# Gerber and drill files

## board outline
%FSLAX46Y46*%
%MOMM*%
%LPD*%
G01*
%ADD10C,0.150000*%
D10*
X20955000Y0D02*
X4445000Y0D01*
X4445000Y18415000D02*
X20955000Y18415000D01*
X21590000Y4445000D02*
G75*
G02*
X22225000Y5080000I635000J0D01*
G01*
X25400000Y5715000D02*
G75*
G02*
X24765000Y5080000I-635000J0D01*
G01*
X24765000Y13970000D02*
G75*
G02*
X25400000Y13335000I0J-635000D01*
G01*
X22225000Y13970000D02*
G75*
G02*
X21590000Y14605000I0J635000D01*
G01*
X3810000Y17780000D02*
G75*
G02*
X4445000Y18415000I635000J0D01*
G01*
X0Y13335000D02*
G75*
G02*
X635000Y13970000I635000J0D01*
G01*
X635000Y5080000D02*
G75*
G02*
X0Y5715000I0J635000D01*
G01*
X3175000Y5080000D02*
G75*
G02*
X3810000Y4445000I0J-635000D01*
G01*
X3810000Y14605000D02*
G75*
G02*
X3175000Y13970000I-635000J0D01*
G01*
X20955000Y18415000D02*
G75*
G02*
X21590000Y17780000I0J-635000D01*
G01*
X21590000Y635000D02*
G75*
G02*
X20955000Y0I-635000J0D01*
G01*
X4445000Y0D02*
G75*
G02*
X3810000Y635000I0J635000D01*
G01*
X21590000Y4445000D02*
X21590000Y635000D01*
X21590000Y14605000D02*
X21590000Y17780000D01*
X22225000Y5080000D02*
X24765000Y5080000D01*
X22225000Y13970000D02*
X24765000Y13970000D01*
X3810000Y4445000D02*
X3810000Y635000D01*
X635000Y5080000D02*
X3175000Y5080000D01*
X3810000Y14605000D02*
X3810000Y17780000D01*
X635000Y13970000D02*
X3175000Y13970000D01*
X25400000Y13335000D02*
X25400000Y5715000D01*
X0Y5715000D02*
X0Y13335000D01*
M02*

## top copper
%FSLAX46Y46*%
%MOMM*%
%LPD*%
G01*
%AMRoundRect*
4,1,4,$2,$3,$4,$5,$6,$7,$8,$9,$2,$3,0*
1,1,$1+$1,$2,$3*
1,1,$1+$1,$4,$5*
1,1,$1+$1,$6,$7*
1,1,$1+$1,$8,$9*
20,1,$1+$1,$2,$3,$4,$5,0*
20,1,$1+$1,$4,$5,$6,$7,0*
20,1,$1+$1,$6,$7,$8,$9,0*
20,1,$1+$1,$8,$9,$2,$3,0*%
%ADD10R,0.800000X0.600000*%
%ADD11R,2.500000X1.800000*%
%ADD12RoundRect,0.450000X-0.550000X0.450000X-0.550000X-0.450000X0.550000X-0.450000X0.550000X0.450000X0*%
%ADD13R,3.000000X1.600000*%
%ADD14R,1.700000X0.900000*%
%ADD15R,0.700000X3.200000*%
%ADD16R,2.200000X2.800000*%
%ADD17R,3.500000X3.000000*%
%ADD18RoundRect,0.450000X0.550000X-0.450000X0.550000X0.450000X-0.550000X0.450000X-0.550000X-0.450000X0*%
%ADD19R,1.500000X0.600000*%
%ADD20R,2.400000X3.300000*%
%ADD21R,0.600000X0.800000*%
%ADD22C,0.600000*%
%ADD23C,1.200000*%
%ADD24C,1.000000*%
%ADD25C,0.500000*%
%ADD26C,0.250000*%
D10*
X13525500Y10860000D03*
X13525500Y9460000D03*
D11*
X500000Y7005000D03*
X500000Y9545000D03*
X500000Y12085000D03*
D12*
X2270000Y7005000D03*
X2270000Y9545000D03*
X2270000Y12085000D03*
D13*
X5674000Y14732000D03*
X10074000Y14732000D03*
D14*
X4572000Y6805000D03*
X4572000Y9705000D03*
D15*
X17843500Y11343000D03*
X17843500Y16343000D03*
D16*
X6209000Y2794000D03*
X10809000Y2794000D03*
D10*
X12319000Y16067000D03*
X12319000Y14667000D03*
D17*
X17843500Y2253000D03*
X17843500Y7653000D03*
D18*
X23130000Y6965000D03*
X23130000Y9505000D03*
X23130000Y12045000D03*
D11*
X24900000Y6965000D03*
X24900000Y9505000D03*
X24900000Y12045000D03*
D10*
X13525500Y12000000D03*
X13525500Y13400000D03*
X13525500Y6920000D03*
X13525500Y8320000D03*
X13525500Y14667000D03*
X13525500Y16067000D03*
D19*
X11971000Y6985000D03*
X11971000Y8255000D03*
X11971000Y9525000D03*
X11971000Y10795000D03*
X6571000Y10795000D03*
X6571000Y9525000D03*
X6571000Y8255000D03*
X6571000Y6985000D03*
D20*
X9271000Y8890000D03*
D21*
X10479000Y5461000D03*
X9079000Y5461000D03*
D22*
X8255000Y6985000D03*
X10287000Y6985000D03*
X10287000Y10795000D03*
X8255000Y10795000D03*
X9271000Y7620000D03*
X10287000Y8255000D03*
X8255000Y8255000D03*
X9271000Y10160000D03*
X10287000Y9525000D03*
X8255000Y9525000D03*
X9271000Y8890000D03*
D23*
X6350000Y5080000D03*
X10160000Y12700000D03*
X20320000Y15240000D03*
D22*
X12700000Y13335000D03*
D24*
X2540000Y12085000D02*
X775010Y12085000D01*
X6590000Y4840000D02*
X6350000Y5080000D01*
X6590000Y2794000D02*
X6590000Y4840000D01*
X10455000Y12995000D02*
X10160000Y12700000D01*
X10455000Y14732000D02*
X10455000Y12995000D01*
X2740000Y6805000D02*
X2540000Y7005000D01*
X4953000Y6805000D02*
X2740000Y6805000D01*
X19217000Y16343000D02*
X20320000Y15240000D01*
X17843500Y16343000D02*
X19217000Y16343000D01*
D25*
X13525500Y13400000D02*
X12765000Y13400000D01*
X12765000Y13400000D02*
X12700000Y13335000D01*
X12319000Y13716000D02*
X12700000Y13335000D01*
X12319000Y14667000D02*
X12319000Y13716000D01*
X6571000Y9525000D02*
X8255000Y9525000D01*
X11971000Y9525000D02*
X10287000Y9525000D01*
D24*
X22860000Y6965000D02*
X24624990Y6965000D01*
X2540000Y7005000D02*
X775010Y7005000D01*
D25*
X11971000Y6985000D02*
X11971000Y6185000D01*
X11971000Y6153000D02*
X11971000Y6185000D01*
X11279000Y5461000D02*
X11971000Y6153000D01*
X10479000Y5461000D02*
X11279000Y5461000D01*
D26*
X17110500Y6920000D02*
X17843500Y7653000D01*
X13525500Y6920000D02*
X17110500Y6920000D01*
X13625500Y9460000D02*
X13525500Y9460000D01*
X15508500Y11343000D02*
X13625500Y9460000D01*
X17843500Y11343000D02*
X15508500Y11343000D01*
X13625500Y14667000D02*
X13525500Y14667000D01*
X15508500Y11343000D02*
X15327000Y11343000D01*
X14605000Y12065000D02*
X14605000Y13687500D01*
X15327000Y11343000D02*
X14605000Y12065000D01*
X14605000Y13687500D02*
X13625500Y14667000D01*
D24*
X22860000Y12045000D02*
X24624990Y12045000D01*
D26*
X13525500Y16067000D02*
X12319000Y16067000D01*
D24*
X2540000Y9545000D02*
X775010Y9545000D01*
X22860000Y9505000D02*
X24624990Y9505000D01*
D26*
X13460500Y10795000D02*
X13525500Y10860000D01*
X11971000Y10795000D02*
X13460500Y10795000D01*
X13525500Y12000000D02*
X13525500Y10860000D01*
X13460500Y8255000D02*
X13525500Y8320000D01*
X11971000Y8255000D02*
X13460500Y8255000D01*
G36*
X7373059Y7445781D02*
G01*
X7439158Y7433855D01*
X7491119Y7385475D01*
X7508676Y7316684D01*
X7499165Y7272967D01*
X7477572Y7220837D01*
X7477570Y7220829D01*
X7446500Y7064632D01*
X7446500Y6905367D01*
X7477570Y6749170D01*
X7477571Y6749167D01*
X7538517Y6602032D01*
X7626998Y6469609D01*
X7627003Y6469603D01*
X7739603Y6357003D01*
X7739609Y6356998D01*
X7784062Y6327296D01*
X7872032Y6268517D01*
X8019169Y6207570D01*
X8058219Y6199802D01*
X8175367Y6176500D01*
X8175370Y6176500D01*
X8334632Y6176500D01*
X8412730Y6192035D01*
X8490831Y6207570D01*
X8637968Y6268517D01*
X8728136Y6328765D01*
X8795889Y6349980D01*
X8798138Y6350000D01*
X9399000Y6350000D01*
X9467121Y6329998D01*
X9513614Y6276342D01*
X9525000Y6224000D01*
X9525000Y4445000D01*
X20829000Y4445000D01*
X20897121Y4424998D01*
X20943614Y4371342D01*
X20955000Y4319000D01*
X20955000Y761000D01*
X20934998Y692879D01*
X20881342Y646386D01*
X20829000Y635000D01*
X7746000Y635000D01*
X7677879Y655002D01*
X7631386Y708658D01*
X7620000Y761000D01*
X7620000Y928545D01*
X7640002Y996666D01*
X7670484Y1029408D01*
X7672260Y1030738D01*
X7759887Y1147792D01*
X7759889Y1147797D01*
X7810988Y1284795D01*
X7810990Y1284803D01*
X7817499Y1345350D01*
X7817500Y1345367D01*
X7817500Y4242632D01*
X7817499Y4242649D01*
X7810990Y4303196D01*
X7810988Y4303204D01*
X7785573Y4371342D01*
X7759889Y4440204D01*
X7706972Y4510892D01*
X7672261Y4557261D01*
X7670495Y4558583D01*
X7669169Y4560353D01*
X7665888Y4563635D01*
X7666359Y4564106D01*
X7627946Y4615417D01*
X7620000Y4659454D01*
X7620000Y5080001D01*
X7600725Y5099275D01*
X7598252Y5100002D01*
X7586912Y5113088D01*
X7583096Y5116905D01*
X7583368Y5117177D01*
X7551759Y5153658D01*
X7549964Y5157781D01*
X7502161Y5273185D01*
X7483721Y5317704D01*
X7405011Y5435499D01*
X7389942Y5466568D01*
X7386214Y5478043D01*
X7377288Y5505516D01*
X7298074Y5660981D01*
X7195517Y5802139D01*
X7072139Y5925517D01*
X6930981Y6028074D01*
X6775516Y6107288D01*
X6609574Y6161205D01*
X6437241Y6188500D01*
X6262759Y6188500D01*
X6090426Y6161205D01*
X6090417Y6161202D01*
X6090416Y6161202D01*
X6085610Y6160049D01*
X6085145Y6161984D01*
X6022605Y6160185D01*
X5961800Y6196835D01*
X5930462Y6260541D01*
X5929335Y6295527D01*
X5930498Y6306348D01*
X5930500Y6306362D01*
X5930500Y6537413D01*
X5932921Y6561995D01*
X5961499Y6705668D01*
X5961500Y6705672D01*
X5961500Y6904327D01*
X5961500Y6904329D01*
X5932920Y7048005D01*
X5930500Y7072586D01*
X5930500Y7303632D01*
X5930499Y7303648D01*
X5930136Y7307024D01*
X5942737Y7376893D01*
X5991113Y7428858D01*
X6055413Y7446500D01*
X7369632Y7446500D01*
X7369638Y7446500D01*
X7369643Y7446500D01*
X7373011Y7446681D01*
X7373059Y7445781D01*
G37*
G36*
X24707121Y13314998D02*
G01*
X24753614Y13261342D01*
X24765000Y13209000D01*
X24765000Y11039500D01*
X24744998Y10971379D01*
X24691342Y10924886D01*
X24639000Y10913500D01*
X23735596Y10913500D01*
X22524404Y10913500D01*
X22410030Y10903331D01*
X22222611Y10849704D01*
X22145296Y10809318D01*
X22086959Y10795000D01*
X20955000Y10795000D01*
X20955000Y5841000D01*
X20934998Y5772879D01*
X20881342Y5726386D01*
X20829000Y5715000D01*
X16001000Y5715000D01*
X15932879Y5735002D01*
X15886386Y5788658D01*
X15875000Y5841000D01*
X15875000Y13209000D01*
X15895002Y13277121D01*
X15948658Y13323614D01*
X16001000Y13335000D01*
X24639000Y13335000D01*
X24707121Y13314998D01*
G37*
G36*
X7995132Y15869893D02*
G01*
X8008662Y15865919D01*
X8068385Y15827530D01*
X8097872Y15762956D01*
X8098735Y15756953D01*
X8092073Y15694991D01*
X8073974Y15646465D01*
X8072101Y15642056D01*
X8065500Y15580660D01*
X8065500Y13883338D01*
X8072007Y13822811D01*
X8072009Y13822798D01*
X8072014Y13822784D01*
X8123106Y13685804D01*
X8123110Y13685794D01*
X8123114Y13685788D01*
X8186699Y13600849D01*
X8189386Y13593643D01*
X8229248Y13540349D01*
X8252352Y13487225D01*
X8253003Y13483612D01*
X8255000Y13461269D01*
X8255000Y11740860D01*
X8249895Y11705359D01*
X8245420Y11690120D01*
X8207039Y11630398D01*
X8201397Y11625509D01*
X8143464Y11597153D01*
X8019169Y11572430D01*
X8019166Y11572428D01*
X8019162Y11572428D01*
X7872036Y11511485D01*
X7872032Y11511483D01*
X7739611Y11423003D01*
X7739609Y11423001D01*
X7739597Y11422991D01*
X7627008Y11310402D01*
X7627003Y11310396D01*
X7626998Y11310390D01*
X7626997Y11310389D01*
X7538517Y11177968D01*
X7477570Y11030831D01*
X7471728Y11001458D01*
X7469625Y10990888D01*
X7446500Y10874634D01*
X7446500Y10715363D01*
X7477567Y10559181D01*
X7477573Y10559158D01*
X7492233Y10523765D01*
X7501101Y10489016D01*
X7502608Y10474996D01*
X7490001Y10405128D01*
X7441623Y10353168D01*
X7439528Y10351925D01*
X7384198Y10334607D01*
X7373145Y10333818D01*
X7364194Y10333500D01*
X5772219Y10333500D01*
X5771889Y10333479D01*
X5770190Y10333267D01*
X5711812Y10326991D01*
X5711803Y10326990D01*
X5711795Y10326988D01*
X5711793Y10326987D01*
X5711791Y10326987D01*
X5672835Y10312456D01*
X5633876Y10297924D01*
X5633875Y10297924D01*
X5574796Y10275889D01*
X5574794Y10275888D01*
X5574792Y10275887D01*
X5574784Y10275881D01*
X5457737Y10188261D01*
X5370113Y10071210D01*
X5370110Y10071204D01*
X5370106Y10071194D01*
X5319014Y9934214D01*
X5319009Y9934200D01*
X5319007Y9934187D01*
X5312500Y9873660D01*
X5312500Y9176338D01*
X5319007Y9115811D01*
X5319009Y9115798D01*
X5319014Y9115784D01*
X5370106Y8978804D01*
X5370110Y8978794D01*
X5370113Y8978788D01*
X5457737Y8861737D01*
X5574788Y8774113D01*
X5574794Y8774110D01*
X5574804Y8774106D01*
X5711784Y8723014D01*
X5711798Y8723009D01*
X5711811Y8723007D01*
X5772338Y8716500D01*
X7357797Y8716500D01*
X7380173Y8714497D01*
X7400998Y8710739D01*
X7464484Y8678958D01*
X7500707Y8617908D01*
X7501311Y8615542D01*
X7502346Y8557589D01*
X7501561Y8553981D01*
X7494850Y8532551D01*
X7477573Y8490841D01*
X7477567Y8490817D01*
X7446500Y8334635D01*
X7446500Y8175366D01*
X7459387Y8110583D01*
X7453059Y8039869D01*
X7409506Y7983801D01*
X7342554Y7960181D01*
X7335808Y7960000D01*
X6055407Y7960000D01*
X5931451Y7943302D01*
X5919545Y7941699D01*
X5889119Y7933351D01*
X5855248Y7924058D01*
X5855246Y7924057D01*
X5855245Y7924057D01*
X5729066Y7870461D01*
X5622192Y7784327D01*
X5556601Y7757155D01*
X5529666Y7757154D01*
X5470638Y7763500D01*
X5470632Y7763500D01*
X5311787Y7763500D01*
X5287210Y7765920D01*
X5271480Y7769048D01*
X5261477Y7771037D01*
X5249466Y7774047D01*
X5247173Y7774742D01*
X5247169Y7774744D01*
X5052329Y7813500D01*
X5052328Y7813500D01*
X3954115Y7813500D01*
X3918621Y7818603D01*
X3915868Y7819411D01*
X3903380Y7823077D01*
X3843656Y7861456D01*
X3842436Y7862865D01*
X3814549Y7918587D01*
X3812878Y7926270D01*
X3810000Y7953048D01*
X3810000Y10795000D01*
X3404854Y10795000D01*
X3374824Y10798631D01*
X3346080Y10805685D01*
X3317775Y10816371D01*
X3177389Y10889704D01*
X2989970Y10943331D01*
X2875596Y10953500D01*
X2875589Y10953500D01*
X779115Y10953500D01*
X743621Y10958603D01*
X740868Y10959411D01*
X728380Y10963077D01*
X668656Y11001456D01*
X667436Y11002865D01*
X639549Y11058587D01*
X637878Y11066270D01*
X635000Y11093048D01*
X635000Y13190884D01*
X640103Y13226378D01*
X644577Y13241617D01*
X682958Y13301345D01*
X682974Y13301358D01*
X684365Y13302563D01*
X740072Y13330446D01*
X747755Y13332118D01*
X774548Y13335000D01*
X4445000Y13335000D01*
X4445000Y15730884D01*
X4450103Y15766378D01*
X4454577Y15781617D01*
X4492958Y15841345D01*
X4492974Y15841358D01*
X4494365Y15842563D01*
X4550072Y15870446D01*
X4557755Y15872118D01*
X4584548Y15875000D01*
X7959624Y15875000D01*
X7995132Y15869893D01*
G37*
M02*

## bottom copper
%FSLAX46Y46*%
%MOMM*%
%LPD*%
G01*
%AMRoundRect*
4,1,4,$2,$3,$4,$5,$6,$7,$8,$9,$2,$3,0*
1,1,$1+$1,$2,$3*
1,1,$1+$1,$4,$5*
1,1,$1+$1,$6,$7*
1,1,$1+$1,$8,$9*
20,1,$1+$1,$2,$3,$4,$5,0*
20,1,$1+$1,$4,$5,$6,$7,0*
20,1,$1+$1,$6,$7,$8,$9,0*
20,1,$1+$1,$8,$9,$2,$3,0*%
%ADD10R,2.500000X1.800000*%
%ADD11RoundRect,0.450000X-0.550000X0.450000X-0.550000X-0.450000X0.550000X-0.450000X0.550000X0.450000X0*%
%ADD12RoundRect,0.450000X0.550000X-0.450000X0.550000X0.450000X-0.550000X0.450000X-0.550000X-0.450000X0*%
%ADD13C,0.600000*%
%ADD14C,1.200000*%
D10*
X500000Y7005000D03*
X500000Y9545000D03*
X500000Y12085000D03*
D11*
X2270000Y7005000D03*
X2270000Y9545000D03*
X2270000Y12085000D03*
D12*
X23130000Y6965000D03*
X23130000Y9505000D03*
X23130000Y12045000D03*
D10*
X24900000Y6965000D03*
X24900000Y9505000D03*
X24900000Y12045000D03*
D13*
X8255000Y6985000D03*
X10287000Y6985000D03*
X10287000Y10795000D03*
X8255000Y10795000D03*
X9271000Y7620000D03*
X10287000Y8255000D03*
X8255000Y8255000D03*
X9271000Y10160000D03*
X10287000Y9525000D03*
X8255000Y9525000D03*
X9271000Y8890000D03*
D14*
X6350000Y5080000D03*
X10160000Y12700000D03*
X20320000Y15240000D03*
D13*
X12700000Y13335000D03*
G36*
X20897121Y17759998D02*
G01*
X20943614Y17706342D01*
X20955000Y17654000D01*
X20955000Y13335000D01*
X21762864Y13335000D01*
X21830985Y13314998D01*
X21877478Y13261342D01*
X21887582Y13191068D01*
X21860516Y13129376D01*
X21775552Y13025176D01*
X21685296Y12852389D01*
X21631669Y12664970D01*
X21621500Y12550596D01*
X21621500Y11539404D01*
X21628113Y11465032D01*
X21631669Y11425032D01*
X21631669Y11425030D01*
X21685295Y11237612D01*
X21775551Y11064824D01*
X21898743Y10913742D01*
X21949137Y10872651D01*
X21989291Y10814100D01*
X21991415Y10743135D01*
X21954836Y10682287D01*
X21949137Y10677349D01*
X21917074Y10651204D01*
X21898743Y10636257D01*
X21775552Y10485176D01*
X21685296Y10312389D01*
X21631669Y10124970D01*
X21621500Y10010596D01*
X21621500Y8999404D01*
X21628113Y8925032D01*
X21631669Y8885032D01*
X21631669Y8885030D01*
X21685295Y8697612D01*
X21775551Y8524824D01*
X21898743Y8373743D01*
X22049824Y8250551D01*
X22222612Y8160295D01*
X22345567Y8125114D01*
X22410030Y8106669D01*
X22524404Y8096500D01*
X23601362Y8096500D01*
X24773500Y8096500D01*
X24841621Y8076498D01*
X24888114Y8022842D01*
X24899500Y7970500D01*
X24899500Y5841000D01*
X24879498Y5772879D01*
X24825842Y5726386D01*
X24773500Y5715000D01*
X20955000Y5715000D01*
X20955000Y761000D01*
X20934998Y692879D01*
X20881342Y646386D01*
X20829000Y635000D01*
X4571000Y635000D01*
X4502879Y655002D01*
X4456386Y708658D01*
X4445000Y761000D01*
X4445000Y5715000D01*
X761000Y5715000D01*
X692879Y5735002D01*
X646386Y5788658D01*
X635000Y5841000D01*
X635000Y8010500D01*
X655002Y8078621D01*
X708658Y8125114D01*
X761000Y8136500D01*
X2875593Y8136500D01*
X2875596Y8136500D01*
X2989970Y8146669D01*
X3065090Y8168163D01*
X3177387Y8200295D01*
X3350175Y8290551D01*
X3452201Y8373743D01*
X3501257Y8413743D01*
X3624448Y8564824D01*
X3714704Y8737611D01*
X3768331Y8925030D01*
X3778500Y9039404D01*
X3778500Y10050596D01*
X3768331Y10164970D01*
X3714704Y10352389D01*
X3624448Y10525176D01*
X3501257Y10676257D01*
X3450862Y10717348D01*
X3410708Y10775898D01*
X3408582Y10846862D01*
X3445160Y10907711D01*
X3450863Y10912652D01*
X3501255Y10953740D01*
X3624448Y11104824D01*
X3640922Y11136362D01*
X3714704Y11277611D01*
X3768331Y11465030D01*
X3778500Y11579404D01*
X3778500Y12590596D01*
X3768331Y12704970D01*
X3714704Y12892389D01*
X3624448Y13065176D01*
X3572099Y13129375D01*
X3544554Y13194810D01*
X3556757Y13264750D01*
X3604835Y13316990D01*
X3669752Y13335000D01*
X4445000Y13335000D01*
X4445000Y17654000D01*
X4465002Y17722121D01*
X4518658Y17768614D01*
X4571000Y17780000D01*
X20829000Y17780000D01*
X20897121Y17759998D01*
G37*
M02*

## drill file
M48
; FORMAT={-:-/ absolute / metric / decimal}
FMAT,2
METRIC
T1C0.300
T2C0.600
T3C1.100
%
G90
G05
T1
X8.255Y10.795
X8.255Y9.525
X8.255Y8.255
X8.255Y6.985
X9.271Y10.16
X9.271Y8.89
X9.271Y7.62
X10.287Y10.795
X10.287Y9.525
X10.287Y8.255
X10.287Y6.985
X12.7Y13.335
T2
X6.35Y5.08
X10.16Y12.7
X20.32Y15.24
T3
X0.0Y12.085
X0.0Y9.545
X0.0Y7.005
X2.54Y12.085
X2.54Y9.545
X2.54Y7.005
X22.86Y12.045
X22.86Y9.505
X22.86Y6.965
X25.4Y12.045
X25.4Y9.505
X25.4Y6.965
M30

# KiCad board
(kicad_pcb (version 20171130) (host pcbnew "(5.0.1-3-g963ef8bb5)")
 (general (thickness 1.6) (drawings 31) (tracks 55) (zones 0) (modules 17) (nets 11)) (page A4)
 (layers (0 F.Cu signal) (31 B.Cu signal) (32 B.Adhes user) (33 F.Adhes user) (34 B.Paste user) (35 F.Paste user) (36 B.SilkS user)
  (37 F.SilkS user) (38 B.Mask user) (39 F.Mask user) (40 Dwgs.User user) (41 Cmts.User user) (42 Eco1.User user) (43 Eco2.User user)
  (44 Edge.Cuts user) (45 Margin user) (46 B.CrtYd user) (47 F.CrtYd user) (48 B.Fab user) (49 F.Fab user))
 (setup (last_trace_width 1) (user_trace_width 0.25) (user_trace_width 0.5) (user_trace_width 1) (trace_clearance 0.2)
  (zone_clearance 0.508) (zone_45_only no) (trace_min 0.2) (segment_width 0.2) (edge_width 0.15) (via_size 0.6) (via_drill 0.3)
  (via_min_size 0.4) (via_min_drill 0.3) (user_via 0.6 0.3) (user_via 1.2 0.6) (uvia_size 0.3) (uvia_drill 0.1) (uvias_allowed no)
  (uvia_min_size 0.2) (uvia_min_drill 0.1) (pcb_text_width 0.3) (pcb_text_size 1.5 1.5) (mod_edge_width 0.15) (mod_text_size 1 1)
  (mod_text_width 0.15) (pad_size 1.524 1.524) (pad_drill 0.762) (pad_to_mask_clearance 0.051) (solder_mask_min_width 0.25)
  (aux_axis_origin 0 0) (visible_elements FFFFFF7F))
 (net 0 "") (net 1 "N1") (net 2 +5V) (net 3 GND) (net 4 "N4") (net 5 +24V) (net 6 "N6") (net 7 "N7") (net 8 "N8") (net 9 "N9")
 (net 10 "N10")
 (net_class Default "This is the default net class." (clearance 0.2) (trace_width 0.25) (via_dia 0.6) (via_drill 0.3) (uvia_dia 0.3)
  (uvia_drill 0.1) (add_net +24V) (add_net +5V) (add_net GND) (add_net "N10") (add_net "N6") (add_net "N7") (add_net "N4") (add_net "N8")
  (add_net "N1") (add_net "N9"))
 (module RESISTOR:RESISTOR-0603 (layer F.Cu) (at 13.5255 -10.16 90)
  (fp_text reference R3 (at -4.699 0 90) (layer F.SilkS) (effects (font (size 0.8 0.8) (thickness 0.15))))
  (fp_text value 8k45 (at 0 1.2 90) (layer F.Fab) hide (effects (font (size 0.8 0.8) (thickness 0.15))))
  (pad 2 smd rect (at 0.7 0 90) (size 0.6 0.8) (layers F.Cu F.Paste F.Mask) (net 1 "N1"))
  (pad 1 smd rect (at -0.7 0 90) (size 0.6 0.8) (layers F.Cu F.Paste F.Mask) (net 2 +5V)))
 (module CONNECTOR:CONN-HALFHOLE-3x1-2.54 (layer F.Cu) (at 1.27 -9.525 270)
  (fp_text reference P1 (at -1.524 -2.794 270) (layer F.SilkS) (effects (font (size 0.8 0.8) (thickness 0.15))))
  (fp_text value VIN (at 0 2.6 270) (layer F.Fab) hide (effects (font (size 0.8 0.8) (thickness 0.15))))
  (pad 3 thru_hole rect (at 2.52 1.27 270) (size 1.8 2.5) (drill 1.1 (offset 0 -0.5)) (layers *.Cu *.Mask) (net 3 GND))
  (pad 2 thru_hole rect (at -0.02 1.27 270) (size 1.8 2.5) (drill 1.1 (offset 0 -0.5)) (layers *.Cu *.Mask) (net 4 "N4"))
  (pad 1 thru_hole rect (at -2.56 1.27 270) (size 1.8 2.5) (drill 1.1 (offset 0 -0.5)) (layers *.Cu *.Mask) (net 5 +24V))
  (pad 3 thru_hole roundrect (at 2.52 -1.27 270) (size 1.8 2) (drill 1.1 (offset 0 0.27)) (layers *.Cu *.Mask) (roundrect_rratio 0.25)
   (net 3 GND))
  (pad 2 thru_hole roundrect (at -0.02 -1.27 270) (size 1.8 2) (drill 1.1 (offset 0 0.27)) (layers *.Cu *.Mask) (roundrect_rratio 0.25)
   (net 4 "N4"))
  (pad 1 thru_hole roundrect (at -2.56 -1.27 270) (size 1.8 2) (drill 1.1 (offset 0 0.27)) (layers *.Cu *.Mask) (roundrect_rratio 0.25)
   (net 5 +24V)))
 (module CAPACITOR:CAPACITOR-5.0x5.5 (layer F.Cu) (at 7.874 -14.732)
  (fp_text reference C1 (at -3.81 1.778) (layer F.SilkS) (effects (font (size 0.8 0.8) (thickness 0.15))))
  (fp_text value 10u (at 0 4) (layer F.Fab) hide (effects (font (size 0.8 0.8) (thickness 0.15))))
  (pad 1 smd rect (at -2.2 0) (size 3 1.6) (layers F.Cu F.Paste F.Mask) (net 5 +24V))
  (pad 2 smd rect (at 2.2 0) (size 3 1.6) (layers F.Cu F.Paste F.Mask) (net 3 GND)))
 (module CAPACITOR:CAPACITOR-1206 (layer F.Cu) (at 4.572 -8.255 270)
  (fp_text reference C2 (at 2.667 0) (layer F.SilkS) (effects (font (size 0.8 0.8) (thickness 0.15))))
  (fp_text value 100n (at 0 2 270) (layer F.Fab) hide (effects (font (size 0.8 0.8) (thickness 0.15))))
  (pad 2 smd rect (at 1.45 0 270) (size 0.9 1.7) (layers F.Cu F.Paste F.Mask) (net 3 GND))
  (pad 1 smd rect (at -1.45 0 270) (size 0.9 1.7) (layers F.Cu F.Paste F.Mask) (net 5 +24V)))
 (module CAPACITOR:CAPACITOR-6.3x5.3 (layer F.Cu) (at 17.8435 -13.843 90)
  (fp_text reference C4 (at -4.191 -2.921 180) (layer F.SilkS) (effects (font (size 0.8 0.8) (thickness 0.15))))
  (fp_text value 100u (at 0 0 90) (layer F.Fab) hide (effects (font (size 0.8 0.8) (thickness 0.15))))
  (pad 1 smd rect (at -2.5 0 90) (size 3.2 0.7) (layers F.Cu F.Paste F.Mask) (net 2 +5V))
  (pad 2 smd rect (at 2.5 0 90) (size 3.2 0.7) (layers F.Cu F.Paste F.Mask) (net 3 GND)))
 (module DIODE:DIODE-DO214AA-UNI (layer F.Cu) (at 8.509 -2.794)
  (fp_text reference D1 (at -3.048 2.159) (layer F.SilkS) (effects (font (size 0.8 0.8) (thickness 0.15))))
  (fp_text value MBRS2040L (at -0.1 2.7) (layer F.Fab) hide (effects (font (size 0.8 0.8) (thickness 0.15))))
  (pad 1 smd rect (at -2.3 0) (size 2.2 2.8) (layers F.Cu F.Paste F.Mask) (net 3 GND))
  (pad 2 smd rect (at 2.3 0) (size 2.2 2.8) (layers F.Cu F.Paste F.Mask) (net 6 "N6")))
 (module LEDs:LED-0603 (layer F.Cu) (at 12.319 -15.367 270)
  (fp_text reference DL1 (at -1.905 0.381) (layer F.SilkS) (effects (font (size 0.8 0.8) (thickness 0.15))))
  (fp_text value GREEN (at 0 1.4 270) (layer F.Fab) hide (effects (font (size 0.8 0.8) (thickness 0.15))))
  (pad 1 smd rect (at -0.7 0 270) (size 0.6 0.8) (layers F.Cu F.Paste F.Mask) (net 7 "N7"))
  (pad 2 smd rect (at 0.7 0 270) (size 0.6 0.8) (layers F.Cu F.Paste F.Mask) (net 3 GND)))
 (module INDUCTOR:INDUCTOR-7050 (layer F.Cu) (at 17.8435 -4.953 90)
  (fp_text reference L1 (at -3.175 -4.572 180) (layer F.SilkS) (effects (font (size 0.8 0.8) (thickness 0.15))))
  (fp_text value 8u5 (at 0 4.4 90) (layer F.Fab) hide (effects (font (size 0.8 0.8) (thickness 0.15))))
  (pad 1 smd rect (at -2.7 0 90) (size 3 3.5) (layers F.Cu F.Paste F.Mask) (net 6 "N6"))
  (pad 2 smd rect (at 2.7 0 90) (size 3 3.5) (layers F.Cu F.Paste F.Mask) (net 2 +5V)))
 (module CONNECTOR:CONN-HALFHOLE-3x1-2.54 (layer F.Cu) (at 24.13 -9.525 90)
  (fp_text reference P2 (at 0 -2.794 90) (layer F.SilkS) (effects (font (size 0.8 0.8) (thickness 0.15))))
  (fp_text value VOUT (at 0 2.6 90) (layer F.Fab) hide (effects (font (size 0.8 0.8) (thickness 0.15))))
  (pad 1 thru_hole roundrect (at -2.56 -1.27 90) (size 1.8 2) (drill 1.1 (offset 0 0.27)) (layers *.Cu *.Mask) (roundrect_rratio 0.25)
   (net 3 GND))
  (pad 2 thru_hole roundrect (at -0.02 -1.27 90) (size 1.8 2) (drill 1.1 (offset 0 0.27)) (layers *.Cu *.Mask) (roundrect_rratio 0.25)
   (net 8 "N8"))
  (pad 3 thru_hole roundrect (at 2.52 -1.27 90) (size 1.8 2) (drill 1.1 (offset 0 0.27)) (layers *.Cu *.Mask) (roundrect_rratio 0.25)
   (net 2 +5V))
  (pad 1 thru_hole rect (at -2.56 1.27 90) (size 1.8 2.5) (drill 1.1 (offset 0 -0.5)) (layers *.Cu *.Mask) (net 3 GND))
  (pad 2 thru_hole rect (at -0.02 1.27 90) (size 1.8 2.5) (drill 1.1 (offset 0 -0.5)) (layers *.Cu *.Mask) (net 8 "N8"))
  (pad 3 thru_hole rect (at 2.52 1.27 90) (size 1.8 2.5) (drill 1.1 (offset 0 -0.5)) (layers *.Cu *.Mask) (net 2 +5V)))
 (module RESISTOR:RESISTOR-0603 (layer F.Cu) (at 13.5255 -12.7 90)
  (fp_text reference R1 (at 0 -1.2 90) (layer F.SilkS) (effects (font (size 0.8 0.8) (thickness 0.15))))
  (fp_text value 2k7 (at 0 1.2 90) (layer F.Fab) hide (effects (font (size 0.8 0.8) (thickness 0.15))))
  (pad 1 smd rect (at -0.7 0 90) (size 0.6 0.8) (layers F.Cu F.Paste F.Mask) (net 1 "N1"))
  (pad 2 smd rect (at 0.7 0 90) (size 0.6 0.8) (layers F.Cu F.Paste F.Mask) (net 3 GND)))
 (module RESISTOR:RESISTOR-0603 (layer F.Cu) (at 13.5255 -7.62 90)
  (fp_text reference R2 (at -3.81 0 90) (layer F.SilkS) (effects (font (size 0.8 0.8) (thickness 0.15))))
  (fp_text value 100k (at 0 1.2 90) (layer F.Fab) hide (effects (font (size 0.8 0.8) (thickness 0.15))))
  (pad 1 smd rect (at -0.7 0 90) (size 0.6 0.8) (layers F.Cu F.Paste F.Mask) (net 2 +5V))
  (pad 2 smd rect (at 0.7 0 90) (size 0.6 0.8) (layers F.Cu F.Paste F.Mask) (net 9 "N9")))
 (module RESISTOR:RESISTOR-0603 (layer F.Cu) (at 13.5255 -15.367 270)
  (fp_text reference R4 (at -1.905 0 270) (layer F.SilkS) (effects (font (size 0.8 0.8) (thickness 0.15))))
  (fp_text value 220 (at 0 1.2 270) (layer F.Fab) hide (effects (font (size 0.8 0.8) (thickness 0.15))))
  (pad 2 smd rect (at 0.7 0 270) (size 0.6 0.8) (layers F.Cu F.Paste F.Mask) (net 2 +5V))
  (pad 1 smd rect (at -0.7 0 270) (size 0.6 0.8) (layers F.Cu F.Paste F.Mask) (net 7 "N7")))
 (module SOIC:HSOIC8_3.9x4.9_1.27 (layer F.Cu) (at 9.271 -8.89 180)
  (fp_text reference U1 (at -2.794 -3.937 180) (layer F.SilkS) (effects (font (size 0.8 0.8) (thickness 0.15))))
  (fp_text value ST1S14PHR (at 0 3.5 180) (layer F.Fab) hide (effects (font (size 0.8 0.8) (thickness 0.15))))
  (pad 1 smd rect (at -2.7 -1.905 180) (size 1.5 0.6) (layers F.Cu F.Paste F.Mask) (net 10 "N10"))
  (pad 2 smd rect (at -2.7 -0.635 180) (size 1.5 0.6) (layers F.Cu F.Paste F.Mask) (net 9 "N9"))
  (pad 3 smd rect (at -2.7 0.635 180) (size 1.5 0.6) (layers F.Cu F.Paste F.Mask) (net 3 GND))
  (pad 4 smd rect (at -2.7 1.905 180) (size 1.5 0.6) (layers F.Cu F.Paste F.Mask) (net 1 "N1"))
  (pad 5 smd rect (at 2.7 1.905 180) (size 1.5 0.6) (layers F.Cu F.Paste F.Mask) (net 5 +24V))
  (pad 6 smd rect (at 2.7 0.635 180) (size 1.5 0.6) (layers F.Cu F.Paste F.Mask) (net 3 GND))
  (pad 7 smd rect (at 2.7 -0.635 180) (size 1.5 0.6) (layers F.Cu F.Paste F.Mask) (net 5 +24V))
  (pad 8 smd rect (at 2.7 -1.905 180) (size 1.5 0.6) (layers F.Cu F.Paste F.Mask) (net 6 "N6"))
  (pad 9 smd rect (at 0 0 180) (size 2.4 3.3) (layers F.Cu F.Paste F.Mask) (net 3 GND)))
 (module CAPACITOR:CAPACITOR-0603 (layer F.Cu) (at 9.779 -5.461 180)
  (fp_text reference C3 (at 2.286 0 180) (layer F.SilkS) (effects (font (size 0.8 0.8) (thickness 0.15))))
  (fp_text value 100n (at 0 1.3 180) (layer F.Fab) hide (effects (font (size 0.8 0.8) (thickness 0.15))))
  (pad 1 smd rect (at -0.7 0 180) (size 0.6 0.8) (layers F.Cu F.Paste F.Mask) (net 10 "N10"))
  (pad 2 smd rect (at 0.7 0 180) (size 0.6 0.8) (layers F.Cu F.Paste F.Mask) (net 6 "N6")))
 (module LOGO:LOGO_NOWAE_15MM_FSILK (layer B.Cu) (at 12.954 -16.51 180)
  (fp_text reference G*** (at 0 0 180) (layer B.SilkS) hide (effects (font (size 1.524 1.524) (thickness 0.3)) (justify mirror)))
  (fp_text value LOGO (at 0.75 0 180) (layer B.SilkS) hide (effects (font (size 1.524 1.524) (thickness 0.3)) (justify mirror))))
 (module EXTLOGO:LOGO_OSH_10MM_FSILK (layer B.Cu) (at 12.7 -9.525 180)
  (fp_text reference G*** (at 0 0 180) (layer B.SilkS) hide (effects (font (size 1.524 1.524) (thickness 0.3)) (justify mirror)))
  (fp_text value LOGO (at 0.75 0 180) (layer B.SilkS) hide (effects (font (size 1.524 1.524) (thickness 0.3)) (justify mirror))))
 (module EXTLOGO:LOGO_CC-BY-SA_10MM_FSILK (layer B.Cu) (at 12.7 -2.032 180)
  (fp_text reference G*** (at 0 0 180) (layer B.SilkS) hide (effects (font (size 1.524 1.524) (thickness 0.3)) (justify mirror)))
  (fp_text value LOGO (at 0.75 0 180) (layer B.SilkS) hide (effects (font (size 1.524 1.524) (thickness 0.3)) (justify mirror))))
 (gr_line (start 20.955 0) (end 4.445 0) (layer Edge.Cuts) (width 0.15))
 (gr_line (start 4.445 -18.415) (end 20.955 -18.415) (layer Edge.Cuts) (width 0.15))
 (gr_arc (start 22.225 -4.445) (end 22.225 -5.08) (angle -90) (layer Edge.Cuts) (width 0.15))
 (gr_arc (start 24.765 -5.715) (end 24.765 -5.08) (angle -90) (layer Edge.Cuts) (width 0.15))
 (gr_arc (start 24.765 -13.335) (end 25.4 -13.335) (angle -90) (layer Edge.Cuts) (width 0.15))
 (gr_arc (start 22.225 -14.605) (end 21.59 -14.605) (angle -90) (layer Edge.Cuts) (width 0.15))
 (gr_arc (start 4.445 -17.78) (end 4.445 -18.415) (angle -90) (layer Edge.Cuts) (width 0.15))
 (gr_arc (start 0.635 -13.335) (end 0.635 -13.97) (angle -90) (layer Edge.Cuts) (width 0.15))
 (gr_arc (start 0.635 -5.715) (end 0 -5.715) (angle -90) (layer Edge.Cuts) (width 0.15))
 (gr_arc (start 3.175 -4.445) (end 3.81 -4.445) (angle -90) (layer Edge.Cuts) (width 0.15))
 (gr_arc (start 3.175 -14.605) (end 3.175 -13.97) (angle -90) (layer Edge.Cuts) (width 0.15))
 (gr_arc (start 20.955 -17.78) (end 21.59 -17.78) (angle -90) (layer Edge.Cuts) (width 0.15))
 (gr_arc (start 20.955 -0.635) (end 20.955 0) (angle -90) (layer Edge.Cuts) (width 0.15))
 (gr_arc (start 4.445 -0.635) (end 3.81 -0.635) (angle -90) (layer Edge.Cuts) (width 0.15))
 (gr_line (start 21.59 -4.445) (end 21.59 -0.635) (layer Edge.Cuts) (width 0.15))
 (gr_line (start 21.59 -14.605) (end 21.59 -17.78) (layer Edge.Cuts) (width 0.15))
 (gr_line (start 22.225 -5.08) (end 24.765 -5.08) (layer Edge.Cuts) (width 0.15))
 (gr_line (start 22.225 -13.97) (end 24.765 -13.97) (layer Edge.Cuts) (width 0.15))
 (gr_line (start 3.81 -4.445) (end 3.81 -0.635) (layer Edge.Cuts) (width 0.15))
 (gr_line (start 0.635 -5.08) (end 3.175 -5.08) (layer Edge.Cuts) (width 0.15))
 (gr_line (start 3.81 -14.605) (end 3.81 -17.78) (layer Edge.Cuts) (width 0.15))
 (gr_line (start 0.635 -13.97) (end 3.175 -13.97) (layer Edge.Cuts) (width 0.15))
 (gr_line (start 25.4 -13.335) (end 25.4 -5.715) (layer Edge.Cuts) (width 0.15))
 (gr_line (start 0 -5.715) (end 0 -13.335) (layer Edge.Cuts) (width 0.15))
 (segment (start 2.54 -12.085) (end 0.77501 -12.085) (width 1) (layer F.Cu) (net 5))
 (via (at 8.255 -6.985) (size 0.6) (drill 0.3) (layers F.Cu B.Cu) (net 3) (status 40000))
 (via (at 10.287 -6.985) (size 0.6) (drill 0.3) (layers F.Cu B.Cu) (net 3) (status 40000))
 (via (at 10.287 -10.795) (size 0.6) (drill 0.3) (layers F.Cu B.Cu) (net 3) (status 40000))
 (via (at 8.255 -10.795) (size 0.6) (drill 0.3) (layers F.Cu B.Cu) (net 3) (status 40000))
 (via (at 9.271 -7.62) (size 0.6) (drill 0.3) (layers F.Cu B.Cu) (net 3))
 (via (at 10.287 -8.255) (size 0.6) (drill 0.3) (layers F.Cu B.Cu) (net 3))
 (via (at 8.255 -8.255) (size 0.6) (drill 0.3) (layers F.Cu B.Cu) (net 3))
 (via (at 9.271 -10.16) (size 0.6) (drill 0.3) (layers F.Cu B.Cu) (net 3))
 (via (at 10.287 -9.525) (size 0.6) (drill 0.3) (layers F.Cu B.Cu) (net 3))
 (via (at 8.255 -9.525) (size 0.6) (drill 0.3) (layers F.Cu B.Cu) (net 3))
 (via (at 9.271 -8.89) (size 0.6) (drill 0.3) (layers F.Cu B.Cu) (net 3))
 (via (at 6.35 -5.08) (size 1.2) (drill 0.6) (layers F.Cu B.Cu) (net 3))
 (segment (start 6.59 -4.84) (end 6.35 -5.08) (width 1) (layer F.Cu) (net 3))
 (segment (start 6.59 -2.794) (end 6.59 -4.84) (width 1) (layer F.Cu) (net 3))
 (segment (start 10.455 -12.995) (end 10.16 -12.7) (width 1) (layer F.Cu) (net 3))
 (via (at 10.16 -12.7) (size 1.2) (drill 0.6) (layers F.Cu B.Cu) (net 3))
 (segment (start 10.455 -14.732) (end 10.455 -12.995) (width 1) (layer F.Cu) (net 3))
 (segment (start 2.74 -6.805) (end 2.54 -7.005) (width 1) (layer F.Cu) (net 3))
 (segment (start 4.953 -6.805) (end 2.74 -6.805) (width 1) (layer F.Cu) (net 3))
 (segment (start 19.217 -16.343) (end 20.32 -15.24) (width 1) (layer F.Cu) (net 3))
 (via (at 20.32 -15.24) (size 1.2) (drill 0.6) (layers F.Cu B.Cu) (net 3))
 (segment (start 17.8435 -16.343) (end 19.217 -16.343) (width 1) (layer F.Cu) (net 3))
 (segment (start 13.5255 -13.4) (end 12.765 -13.4) (width 0.5) (layer F.Cu) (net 3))
 (via (at 12.7 -13.335) (size 0.6) (drill 0.3) (layers F.Cu B.Cu) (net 3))
 (segment (start 12.765 -13.4) (end 12.7 -13.335) (width 0.5) (layer F.Cu) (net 3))
 (segment (start 12.319 -13.716) (end 12.7 -13.335) (width 0.5) (layer F.Cu) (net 3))
 (segment (start 12.319 -14.667) (end 12.319 -13.716) (width 0.5) (layer F.Cu) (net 3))
 (segment (start 6.571 -9.525) (end 8.255 -9.525) (width 0.5) (layer F.Cu) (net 3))
 (segment (start 11.971 -9.525) (end 10.287 -9.525) (width 0.5) (layer F.Cu) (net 3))
 (segment (start 22.86 -6.965) (end 24.62499 -6.965) (width 1) (layer F.Cu) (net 3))
 (segment (start 2.54 -7.005) (end 0.77501 -7.005) (width 1) (layer F.Cu) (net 3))
 (segment (start 11.971 -6.985) (end 11.971 -6.185) (width 0.5) (layer F.Cu) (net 10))
 (segment (start 11.971 -6.153) (end 11.971 -6.185) (width 0.5) (layer F.Cu) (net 10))
 (segment (start 11.279 -5.461) (end 11.971 -6.153) (width 0.5) (layer F.Cu) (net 10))
 (segment (start 10.479 -5.461) (end 11.279 -5.461) (width 0.5) (layer F.Cu) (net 10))
 (segment (start 17.1105 -6.92) (end 17.8435 -7.653) (width 0.25) (layer F.Cu) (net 2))
 (segment (start 13.5255 -6.92) (end 17.1105 -6.92) (width 0.25) (layer F.Cu) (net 2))
 (segment (start 13.6255 -9.46) (end 13.5255 -9.46) (width 0.25) (layer F.Cu) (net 2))
 (segment (start 15.5085 -11.343) (end 13.6255 -9.46) (width 0.25) (layer F.Cu) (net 2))
 (segment (start 17.8435 -11.343) (end 15.5085 -11.343) (width 0.25) (layer F.Cu) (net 2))
 (segment (start 13.6255 -14.667) (end 13.5255 -14.667) (width 0.25) (layer F.Cu) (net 2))
 (segment (start 15.5085 -11.343) (end 15.327 -11.343) (width 0.25) (layer F.Cu) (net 2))
 (segment (start 14.605 -12.065) (end 14.605 -13.6875) (width 0.25) (layer F.Cu) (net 2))
 (segment (start 15.327 -11.343) (end 14.605 -12.065) (width 0.25) (layer F.Cu) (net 2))
 (segment (start 14.605 -13.6875) (end 13.6255 -14.667) (width 0.25) (layer F.Cu) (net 2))
 (segment (start 22.86 -12.045) (end 24.62499 -12.045) (width 1) (layer F.Cu) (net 2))
 (segment (start 13.5255 -16.067) (end 12.319 -16.067) (width 0.25) (layer F.Cu) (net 7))
 (segment (start 2.54 -9.545) (end 0.77501 -9.545) (width 1) (layer F.Cu) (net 4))
 (segment (start 22.86 -9.505) (end 24.62499 -9.505) (width 1) (layer F.Cu) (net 8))
 (segment (start 13.4605 -10.795) (end 13.5255 -10.86) (width 0.25) (layer F.Cu) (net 1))
 (segment (start 11.971 -10.795) (end 13.4605 -10.795) (width 0.25) (layer F.Cu) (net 1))
 (segment (start 13.5255 -12) (end 13.5255 -10.86) (width 0.25) (layer F.Cu) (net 1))
 (segment (start 13.4605 -8.255) (end 13.5255 -8.32) (width 0.25) (layer F.Cu) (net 9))
 (segment (start 11.971 -8.255) (end 13.4605 -8.255) (width 0.25) (layer F.Cu) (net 9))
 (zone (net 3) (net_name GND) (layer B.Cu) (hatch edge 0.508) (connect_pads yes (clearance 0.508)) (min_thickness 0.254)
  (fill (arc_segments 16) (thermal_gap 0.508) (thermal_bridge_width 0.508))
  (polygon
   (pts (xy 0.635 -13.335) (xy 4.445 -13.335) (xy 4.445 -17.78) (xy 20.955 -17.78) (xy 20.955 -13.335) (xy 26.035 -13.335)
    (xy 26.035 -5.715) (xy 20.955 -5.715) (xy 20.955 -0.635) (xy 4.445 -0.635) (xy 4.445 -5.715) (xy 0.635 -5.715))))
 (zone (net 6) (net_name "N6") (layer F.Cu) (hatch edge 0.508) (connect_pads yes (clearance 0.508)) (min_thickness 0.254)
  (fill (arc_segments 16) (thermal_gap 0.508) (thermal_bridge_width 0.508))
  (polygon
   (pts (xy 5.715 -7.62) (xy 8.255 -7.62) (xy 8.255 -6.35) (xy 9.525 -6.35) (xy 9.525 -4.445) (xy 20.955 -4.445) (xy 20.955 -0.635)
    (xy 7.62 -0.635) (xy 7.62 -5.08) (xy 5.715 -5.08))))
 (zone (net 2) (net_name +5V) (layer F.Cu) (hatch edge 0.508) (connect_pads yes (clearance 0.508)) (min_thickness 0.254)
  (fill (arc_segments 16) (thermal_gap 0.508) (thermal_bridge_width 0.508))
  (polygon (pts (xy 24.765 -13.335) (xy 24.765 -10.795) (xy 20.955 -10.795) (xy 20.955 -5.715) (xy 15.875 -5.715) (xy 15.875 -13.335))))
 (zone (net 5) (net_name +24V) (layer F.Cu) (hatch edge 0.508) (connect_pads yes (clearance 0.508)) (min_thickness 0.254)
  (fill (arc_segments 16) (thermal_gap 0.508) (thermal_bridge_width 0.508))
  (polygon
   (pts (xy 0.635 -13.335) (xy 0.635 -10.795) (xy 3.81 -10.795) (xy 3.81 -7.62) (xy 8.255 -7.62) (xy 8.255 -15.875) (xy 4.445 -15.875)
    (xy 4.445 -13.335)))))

